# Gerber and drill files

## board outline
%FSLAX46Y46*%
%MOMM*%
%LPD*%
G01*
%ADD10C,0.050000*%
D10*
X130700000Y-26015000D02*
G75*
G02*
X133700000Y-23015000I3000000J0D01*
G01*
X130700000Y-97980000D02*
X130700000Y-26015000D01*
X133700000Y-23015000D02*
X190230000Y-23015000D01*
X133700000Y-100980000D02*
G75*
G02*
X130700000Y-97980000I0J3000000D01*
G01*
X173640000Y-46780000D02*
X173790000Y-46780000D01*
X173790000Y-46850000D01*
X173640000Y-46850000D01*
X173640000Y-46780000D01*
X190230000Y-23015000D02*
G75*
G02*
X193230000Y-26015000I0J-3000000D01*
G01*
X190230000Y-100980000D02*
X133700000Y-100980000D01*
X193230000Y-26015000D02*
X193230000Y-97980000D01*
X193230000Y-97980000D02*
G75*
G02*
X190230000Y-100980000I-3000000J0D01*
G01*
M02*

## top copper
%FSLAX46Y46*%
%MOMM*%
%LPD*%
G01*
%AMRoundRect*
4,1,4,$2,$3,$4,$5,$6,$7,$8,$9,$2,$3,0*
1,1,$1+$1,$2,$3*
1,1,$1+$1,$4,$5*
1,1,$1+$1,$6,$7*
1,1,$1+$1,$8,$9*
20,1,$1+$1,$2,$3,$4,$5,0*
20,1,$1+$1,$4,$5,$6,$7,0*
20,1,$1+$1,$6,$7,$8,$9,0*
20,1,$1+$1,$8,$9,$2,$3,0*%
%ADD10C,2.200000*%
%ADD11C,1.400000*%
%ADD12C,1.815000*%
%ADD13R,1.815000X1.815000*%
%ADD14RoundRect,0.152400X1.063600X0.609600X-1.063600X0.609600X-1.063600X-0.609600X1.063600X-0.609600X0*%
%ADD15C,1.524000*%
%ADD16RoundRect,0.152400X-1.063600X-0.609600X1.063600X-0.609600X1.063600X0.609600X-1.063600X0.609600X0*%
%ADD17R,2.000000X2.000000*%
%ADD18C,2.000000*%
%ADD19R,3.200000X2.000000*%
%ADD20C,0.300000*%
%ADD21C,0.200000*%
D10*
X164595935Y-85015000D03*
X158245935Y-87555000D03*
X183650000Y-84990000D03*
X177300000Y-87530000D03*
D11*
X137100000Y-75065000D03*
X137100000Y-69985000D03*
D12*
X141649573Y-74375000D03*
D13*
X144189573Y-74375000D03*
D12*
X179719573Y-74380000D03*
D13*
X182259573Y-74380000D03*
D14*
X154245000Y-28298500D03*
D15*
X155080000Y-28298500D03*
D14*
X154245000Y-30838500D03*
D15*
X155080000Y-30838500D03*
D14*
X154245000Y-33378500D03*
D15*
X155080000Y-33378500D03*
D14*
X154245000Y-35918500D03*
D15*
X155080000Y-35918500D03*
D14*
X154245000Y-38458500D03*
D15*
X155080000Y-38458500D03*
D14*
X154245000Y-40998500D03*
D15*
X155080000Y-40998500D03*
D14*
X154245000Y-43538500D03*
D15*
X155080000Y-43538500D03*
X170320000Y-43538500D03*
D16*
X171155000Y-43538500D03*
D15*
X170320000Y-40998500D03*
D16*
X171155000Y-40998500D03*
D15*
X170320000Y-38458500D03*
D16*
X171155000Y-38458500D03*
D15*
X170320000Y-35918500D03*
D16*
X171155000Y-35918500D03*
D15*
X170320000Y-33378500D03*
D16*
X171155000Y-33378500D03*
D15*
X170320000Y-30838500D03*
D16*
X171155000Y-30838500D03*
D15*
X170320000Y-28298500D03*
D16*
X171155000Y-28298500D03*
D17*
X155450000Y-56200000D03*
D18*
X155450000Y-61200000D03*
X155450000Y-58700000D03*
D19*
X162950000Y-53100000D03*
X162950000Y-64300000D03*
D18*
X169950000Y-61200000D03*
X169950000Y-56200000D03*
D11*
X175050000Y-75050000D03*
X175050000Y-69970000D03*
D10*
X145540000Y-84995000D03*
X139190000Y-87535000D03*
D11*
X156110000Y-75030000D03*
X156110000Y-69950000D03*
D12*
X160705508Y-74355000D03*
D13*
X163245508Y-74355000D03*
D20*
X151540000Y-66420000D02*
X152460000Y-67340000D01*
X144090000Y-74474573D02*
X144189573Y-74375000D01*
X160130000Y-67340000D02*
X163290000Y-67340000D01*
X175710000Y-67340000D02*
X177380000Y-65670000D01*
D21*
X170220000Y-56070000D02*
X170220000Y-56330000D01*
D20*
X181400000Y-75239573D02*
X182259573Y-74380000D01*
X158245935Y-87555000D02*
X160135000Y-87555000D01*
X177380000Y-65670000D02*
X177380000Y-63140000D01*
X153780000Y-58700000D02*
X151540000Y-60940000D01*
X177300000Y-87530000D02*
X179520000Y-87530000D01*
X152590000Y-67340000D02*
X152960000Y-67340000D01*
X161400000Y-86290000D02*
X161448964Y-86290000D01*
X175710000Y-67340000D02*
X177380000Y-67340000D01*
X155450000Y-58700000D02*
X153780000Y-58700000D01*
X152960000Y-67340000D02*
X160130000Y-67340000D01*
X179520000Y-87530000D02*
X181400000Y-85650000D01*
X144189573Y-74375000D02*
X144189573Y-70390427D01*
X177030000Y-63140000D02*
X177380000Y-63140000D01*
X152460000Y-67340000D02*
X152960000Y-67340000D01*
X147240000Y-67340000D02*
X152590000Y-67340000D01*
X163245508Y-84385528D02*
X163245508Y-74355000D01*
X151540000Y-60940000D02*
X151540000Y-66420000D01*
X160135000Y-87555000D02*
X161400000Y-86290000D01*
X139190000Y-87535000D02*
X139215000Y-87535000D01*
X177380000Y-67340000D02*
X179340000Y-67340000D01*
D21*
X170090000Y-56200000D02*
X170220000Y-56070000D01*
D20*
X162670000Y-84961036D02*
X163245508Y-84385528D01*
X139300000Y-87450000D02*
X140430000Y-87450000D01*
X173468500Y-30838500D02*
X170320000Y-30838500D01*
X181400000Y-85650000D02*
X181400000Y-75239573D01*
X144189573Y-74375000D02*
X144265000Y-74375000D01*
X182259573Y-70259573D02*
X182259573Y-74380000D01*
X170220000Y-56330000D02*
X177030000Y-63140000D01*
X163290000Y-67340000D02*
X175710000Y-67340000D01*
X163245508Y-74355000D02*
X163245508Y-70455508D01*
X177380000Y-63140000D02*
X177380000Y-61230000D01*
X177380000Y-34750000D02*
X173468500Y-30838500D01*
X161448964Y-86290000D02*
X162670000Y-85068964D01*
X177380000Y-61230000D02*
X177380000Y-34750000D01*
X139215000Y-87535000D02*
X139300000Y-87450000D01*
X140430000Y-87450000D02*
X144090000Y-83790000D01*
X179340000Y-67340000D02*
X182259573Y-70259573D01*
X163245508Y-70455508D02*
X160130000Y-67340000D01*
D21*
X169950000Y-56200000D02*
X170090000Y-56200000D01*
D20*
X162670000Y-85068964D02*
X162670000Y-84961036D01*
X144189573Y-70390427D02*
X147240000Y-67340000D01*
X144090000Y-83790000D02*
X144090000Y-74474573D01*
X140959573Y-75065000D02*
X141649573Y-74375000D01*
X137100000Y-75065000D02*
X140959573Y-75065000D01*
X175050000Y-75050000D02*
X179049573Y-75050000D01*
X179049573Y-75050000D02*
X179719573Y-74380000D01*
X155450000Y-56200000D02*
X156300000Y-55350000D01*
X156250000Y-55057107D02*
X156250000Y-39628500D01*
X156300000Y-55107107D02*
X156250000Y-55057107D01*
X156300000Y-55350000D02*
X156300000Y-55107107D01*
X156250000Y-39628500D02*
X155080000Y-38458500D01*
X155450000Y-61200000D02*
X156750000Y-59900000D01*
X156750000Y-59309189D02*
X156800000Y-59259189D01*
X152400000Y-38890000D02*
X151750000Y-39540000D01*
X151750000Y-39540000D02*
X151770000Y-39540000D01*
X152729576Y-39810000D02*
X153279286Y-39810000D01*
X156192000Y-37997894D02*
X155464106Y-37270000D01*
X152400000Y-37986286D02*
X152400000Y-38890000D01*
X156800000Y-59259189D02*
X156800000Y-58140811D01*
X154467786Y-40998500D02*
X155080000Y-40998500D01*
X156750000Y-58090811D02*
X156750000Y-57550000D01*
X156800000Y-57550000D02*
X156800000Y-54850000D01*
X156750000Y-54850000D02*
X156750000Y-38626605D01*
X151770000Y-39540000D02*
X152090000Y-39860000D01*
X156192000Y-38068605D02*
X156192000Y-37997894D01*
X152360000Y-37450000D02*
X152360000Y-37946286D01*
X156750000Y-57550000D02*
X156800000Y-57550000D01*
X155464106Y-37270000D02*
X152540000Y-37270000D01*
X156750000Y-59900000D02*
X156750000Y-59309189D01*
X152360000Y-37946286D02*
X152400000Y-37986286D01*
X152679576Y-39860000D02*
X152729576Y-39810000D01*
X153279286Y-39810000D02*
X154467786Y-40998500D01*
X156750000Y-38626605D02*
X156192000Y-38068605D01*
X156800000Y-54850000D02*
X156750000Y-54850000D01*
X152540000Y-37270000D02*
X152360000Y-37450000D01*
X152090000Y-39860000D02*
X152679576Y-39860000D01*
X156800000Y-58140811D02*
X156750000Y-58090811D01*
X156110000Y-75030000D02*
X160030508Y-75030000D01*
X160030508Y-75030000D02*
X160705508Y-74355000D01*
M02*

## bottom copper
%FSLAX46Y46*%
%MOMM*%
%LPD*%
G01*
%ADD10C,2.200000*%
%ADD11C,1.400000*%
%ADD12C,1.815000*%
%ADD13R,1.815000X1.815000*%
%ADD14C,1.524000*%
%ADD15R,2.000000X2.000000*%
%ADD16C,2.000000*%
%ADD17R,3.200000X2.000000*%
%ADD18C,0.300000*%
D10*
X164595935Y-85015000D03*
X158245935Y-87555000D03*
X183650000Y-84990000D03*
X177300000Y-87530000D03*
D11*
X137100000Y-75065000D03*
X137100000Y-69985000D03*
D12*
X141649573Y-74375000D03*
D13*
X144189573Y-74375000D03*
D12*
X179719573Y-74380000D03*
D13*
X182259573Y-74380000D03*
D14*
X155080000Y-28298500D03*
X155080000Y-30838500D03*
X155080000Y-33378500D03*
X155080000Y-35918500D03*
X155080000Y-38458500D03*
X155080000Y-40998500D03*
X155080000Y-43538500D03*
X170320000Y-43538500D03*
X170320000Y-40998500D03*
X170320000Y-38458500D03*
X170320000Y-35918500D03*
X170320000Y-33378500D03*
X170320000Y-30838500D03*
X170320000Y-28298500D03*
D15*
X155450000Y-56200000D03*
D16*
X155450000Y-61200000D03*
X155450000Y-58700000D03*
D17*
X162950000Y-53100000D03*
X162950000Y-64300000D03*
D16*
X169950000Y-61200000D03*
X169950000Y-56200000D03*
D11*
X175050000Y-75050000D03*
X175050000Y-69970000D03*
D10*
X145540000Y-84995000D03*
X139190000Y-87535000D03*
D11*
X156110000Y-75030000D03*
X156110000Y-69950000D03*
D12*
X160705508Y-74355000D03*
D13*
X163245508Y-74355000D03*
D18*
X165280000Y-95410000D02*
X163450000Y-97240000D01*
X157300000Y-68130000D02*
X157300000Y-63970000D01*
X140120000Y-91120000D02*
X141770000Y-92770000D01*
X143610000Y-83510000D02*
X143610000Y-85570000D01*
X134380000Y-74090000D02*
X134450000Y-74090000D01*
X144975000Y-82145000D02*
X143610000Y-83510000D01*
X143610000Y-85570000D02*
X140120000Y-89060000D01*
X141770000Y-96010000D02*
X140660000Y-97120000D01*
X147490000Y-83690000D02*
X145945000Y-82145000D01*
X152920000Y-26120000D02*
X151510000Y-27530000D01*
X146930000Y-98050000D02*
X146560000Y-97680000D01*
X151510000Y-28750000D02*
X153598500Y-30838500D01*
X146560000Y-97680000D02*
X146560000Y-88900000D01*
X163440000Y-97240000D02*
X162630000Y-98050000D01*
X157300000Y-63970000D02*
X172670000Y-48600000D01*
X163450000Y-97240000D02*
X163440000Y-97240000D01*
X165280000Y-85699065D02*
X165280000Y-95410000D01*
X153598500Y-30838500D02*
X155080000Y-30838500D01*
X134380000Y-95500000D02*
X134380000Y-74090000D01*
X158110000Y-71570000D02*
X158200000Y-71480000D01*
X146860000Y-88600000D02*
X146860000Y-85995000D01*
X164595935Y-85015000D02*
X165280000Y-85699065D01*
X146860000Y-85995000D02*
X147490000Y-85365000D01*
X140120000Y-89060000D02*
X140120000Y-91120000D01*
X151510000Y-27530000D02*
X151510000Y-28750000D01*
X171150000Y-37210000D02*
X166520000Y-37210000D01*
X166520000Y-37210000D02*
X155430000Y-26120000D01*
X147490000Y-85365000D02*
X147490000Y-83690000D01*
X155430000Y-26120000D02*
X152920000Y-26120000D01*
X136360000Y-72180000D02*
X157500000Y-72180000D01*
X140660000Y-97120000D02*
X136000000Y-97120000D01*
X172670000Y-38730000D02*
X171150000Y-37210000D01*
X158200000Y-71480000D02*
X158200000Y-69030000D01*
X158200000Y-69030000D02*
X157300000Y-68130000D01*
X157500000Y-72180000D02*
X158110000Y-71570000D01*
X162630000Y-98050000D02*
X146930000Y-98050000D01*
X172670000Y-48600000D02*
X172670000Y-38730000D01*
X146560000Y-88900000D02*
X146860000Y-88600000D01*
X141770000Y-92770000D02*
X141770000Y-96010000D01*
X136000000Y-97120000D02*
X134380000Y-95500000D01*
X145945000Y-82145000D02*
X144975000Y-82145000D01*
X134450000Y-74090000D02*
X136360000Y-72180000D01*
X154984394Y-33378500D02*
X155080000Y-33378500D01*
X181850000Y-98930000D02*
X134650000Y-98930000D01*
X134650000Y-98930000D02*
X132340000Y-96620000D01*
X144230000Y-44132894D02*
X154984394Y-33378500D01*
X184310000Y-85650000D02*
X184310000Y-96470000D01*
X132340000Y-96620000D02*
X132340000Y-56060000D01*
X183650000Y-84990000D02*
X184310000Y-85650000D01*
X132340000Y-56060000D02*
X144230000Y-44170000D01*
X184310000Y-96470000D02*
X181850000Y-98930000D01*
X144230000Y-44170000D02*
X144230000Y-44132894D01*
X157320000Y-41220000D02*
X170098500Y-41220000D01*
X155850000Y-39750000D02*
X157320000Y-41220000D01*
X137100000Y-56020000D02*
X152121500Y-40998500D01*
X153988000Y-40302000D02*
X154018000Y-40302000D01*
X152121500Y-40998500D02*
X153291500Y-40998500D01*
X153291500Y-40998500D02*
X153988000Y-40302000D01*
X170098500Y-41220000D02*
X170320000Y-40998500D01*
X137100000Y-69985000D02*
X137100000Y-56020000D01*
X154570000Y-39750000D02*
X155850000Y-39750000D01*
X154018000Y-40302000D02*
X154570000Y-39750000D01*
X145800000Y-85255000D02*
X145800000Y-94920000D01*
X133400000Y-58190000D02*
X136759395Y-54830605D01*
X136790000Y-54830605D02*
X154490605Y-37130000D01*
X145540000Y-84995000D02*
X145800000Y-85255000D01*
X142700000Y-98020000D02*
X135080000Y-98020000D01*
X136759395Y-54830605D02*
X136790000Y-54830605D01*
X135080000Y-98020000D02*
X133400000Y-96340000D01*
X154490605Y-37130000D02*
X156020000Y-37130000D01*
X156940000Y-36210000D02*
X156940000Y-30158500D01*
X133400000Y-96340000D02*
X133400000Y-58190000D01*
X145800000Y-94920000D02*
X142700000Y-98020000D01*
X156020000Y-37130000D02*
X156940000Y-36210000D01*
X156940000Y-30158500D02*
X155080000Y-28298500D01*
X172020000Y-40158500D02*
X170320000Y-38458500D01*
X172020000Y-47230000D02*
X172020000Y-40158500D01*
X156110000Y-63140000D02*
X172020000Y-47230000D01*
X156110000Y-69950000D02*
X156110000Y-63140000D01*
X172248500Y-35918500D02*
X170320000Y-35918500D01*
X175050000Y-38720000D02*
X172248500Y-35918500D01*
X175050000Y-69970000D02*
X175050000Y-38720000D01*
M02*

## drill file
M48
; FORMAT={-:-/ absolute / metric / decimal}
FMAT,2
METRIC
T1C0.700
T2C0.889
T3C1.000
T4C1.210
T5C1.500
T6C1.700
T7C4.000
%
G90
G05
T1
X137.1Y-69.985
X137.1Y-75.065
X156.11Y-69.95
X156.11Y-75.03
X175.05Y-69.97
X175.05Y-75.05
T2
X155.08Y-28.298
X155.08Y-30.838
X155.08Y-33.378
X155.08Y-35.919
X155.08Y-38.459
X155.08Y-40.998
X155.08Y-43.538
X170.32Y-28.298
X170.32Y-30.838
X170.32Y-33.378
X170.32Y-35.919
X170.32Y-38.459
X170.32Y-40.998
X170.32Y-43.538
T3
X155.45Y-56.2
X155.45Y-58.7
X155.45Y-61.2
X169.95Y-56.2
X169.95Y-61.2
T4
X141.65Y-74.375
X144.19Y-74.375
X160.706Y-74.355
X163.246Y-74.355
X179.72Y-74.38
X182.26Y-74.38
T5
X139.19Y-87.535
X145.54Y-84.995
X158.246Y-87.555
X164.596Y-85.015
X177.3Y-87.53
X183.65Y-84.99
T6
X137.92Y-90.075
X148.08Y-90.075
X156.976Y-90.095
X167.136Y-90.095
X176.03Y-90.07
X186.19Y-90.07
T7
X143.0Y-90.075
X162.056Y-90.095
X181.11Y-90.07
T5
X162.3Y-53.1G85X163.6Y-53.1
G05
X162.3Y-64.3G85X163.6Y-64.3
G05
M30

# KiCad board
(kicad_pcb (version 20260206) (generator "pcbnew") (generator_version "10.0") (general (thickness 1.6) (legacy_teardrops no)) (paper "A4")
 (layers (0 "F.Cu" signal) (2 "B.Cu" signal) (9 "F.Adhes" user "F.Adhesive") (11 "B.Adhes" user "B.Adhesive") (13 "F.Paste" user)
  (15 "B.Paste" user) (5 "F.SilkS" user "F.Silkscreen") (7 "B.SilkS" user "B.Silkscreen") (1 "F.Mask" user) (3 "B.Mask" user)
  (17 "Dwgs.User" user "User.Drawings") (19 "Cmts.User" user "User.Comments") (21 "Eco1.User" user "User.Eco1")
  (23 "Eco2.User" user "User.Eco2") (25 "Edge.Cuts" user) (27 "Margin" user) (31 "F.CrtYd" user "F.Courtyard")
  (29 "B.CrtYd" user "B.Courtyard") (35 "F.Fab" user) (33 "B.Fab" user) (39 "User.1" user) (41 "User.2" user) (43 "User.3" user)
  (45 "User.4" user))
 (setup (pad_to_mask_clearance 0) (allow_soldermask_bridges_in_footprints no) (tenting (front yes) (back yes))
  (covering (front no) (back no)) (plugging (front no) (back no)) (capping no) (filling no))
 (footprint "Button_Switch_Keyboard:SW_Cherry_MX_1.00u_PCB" (layer "F.Cu") (at 164.595935 85.015)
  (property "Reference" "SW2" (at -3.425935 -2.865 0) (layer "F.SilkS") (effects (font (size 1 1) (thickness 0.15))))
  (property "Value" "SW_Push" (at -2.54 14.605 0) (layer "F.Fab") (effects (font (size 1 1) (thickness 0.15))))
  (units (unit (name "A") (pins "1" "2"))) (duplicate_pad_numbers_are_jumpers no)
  (pad "" np_thru_hole circle (at -7.62 5.08) (size 1.7 1.7) (drill 1.7) (layers "*.Cu" "*.Mask"))
  (pad "" np_thru_hole circle (at -2.54 5.08) (size 4 4) (drill 4) (layers "*.Cu" "*.Mask"))
  (pad "" np_thru_hole circle (at 2.54 5.08) (size 1.7 1.7) (drill 1.7) (layers "*.Cu" "*.Mask"))
  (pad "1" thru_hole circle (at 0 0) (size 2.2 2.2) (drill 1.5) (layers "*.Cu" "*.Mask") (remove_unused_layers no) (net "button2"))
  (pad "2" thru_hole circle (at -6.35 2.54) (size 2.2 2.2) (drill 1.5) (layers "*.Cu" "*.Mask") (remove_unused_layers no) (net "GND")))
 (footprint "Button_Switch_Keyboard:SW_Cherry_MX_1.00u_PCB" (layer "F.Cu") (at 183.65 84.99)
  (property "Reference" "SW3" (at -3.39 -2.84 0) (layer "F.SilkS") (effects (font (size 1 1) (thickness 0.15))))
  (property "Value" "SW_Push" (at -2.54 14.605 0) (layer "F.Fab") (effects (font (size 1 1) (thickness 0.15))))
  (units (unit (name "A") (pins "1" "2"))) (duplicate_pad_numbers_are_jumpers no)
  (pad "" np_thru_hole circle (at -7.62 5.08) (size 1.7 1.7) (drill 1.7) (layers "*.Cu" "*.Mask"))
  (pad "" np_thru_hole circle (at -2.54 5.08) (size 4 4) (drill 4) (layers "*.Cu" "*.Mask"))
  (pad "" np_thru_hole circle (at 2.54 5.08) (size 1.7 1.7) (drill 1.7) (layers "*.Cu" "*.Mask"))
  (pad "1" thru_hole circle (at 0 0) (size 2.2 2.2) (drill 1.5) (layers "*.Cu" "*.Mask") (remove_unused_layers no) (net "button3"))
  (pad "2" thru_hole circle (at -6.35 2.54) (size 2.2 2.2) (drill 1.5) (layers "*.Cu" "*.Mask") (remove_unused_layers no) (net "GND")))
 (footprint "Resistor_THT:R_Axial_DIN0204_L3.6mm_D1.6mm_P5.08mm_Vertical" (layer "F.Cu") (at 137.1 75.065 90)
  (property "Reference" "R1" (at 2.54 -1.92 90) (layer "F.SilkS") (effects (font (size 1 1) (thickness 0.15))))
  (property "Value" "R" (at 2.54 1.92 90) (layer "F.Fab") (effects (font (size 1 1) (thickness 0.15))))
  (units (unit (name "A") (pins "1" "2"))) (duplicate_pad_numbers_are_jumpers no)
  (pad "1" thru_hole circle (at 0 0 90) (size 1.4 1.4) (drill 0.7) (layers "*.Cu" "*.Mask") (remove_unused_layers no) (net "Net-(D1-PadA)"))
  (pad "2" thru_hole circle (at 5.08 0 90) (size 1.4 1.4) (drill 0.7) (layers "*.Cu" "*.Mask") (remove_unused_layers no) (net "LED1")))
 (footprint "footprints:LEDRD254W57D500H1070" (layer "F.Cu") (at 142.919573 74.375 180)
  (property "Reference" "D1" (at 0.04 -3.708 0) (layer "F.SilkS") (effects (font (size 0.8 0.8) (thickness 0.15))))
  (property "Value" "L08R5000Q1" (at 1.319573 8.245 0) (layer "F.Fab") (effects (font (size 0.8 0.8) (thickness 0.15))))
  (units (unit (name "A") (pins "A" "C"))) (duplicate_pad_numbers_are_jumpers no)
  (pad "A" thru_hole circle (at 1.27 0 180) (size 1.815 1.815) (drill 1.21) (layers "*.Cu" "*.Mask") (remove_unused_layers no)
   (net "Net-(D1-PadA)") (solder_mask_margin 0.102))
  (pad "C" thru_hole rect (at -1.27 0 180) (size 1.815 1.815) (drill 1.21) (layers "*.Cu" "*.Mask") (remove_unused_layers no) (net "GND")
   (solder_mask_margin 0.102)))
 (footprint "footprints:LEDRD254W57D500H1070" (layer "F.Cu") (at 180.989573 74.38 180)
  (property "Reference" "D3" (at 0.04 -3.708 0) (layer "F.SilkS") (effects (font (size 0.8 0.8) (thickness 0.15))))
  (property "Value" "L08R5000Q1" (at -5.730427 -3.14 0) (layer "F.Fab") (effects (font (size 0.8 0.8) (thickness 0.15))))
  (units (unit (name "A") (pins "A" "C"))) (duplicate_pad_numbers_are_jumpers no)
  (pad "A" thru_hole circle (at 1.27 0 180) (size 1.815 1.815) (drill 1.21) (layers "*.Cu" "*.Mask") (remove_unused_layers no)
   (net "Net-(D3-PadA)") (solder_mask_margin 0.102))
  (pad "C" thru_hole rect (at -1.27 0 180) (size 1.815 1.815) (drill 1.21) (layers "*.Cu" "*.Mask") (remove_unused_layers no) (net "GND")
   (solder_mask_margin 0.102)))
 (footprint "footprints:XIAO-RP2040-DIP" (layer "F.Cu") (at 162.7 35.9185 90)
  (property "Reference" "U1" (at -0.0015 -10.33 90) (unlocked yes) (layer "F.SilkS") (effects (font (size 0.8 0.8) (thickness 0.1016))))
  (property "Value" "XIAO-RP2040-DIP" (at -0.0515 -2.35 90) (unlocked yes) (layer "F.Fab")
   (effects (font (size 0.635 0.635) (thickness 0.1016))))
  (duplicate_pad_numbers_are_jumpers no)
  (pad "1" smd roundrect (at 7.62 -8.455 180) (size 2.432 1.524) (layers "F.Cu" "F.Mask") (roundrect_rratio 0.1) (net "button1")
   (thermal_bridge_angle 45))
  (pad "1" thru_hole circle (at 7.62 -7.62 180) (size 1.524 1.524) (drill 0.889) (layers "*.Cu" "*.Mask") (remove_unused_layers no)
   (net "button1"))
  (pad "2" smd roundrect (at 5.08 -8.455 180) (size 2.432 1.524) (layers "F.Cu" "F.Mask") (roundrect_rratio 0.1) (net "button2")
   (thermal_bridge_angle 45))
  (pad "2" thru_hole circle (at 5.08 -7.62 180) (size 1.524 1.524) (drill 0.889) (layers "*.Cu" "*.Mask") (remove_unused_layers no)
   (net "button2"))
  (pad "3" smd roundrect (at 2.54 -8.455 180) (size 2.432 1.524) (layers "F.Cu" "F.Mask") (roundrect_rratio 0.1) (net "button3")
   (thermal_bridge_angle 45))
  (pad "3" thru_hole circle (at 2.54 -7.62 180) (size 1.524 1.524) (drill 0.889) (layers "*.Cu" "*.Mask") (remove_unused_layers no)
   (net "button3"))
  (pad "4" smd roundrect (at 0 -8.455 180) (size 2.432 1.524) (layers "F.Cu" "F.Mask") (roundrect_rratio 0.1)
   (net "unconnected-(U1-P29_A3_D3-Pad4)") (thermal_bridge_angle 45))
  (pad "4" thru_hole circle (at 0 -7.62 180) (size 1.524 1.524) (drill 0.889) (layers "*.Cu" "*.Mask") (remove_unused_layers no)
   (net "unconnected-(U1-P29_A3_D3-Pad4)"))
  (pad "5" smd roundrect (at -2.54 -8.455 180) (size 2.432 1.524) (layers "F.Cu" "F.Mask") (roundrect_rratio 0.1) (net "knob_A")
   (thermal_bridge_angle 45))
  (pad "5" thru_hole circle (at -2.54 -7.62 180) (size 1.524 1.524) (drill 0.889) (layers "*.Cu" "*.Mask") (remove_unused_layers no)
   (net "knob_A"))
  (pad "6" smd roundrect (at -5.08 -8.455 180) (size 2.432 1.524) (layers "F.Cu" "F.Mask") (roundrect_rratio 0.1) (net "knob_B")
   (thermal_bridge_angle 45))
  (pad "6" thru_hole circle (at -5.08 -7.62 180) (size 1.524 1.524) (drill 0.889) (layers "*.Cu" "*.Mask") (remove_unused_layers no)
   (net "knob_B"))
  (pad "7" smd roundrect (at -7.62 -8.455 180) (size 2.432 1.524) (layers "F.Cu" "F.Mask") (roundrect_rratio 0.1)
   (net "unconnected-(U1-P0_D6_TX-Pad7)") (thermal_bridge_angle 45))
  (pad "7" thru_hole circle (at -7.62 -7.62 180) (size 1.524 1.524) (drill 0.889) (layers "*.Cu" "*.Mask") (remove_unused_layers no)
   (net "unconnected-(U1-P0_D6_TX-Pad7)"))
  (pad "8" thru_hole circle (at -7.62 7.62) (size 1.524 1.524) (drill 0.889) (layers "*.Cu" "*.Mask") (remove_unused_layers no)
   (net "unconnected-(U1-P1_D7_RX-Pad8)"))
  (pad "8" smd roundrect (at -7.62 8.455) (size 2.432 1.524) (layers "F.Cu" "F.Mask") (roundrect_rratio 0.1)
   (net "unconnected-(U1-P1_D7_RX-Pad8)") (thermal_bridge_angle 45))
  (pad "9" thru_hole circle (at -5.08 7.62) (size 1.524 1.524) (drill 0.889) (layers "*.Cu" "*.Mask") (remove_unused_layers no) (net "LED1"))
  (pad "9" smd roundrect (at -5.08 8.455) (size 2.432 1.524) (layers "F.Cu" "F.Mask") (roundrect_rratio 0.1) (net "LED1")
   (thermal_bridge_angle 45))
  (pad "10" thru_hole circle (at -2.54 7.62) (size 1.524 1.524) (drill 0.889) (layers "*.Cu" "*.Mask") (remove_unused_layers no)
   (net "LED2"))
  (pad "10" smd roundrect (at -2.54 8.455) (size 2.432 1.524) (layers "F.Cu" "F.Mask") (roundrect_rratio 0.1) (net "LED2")
   (thermal_bridge_angle 45))
  (pad "11" thru_hole circle (at 0 7.62) (size 1.524 1.524) (drill 0.889) (layers "*.Cu" "*.Mask") (remove_unused_layers no) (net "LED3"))
  (pad "11" smd roundrect (at 0 8.455) (size 2.432 1.524) (layers "F.Cu" "F.Mask") (roundrect_rratio 0.1) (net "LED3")
   (thermal_bridge_angle 45))
  (pad "12" thru_hole circle (at 2.54 7.62) (size 1.524 1.524) (drill 0.889) (layers "*.Cu" "*.Mask") (remove_unused_layers no)
   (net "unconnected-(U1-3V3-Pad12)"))
  (pad "12" smd roundrect (at 2.54 8.455) (size 2.432 1.524) (layers "F.Cu" "F.Mask") (roundrect_rratio 0.1)
   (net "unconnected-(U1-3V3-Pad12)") (thermal_bridge_angle 45))
  (pad "13" thru_hole circle (at 5.08 7.62) (size 1.524 1.524) (drill 0.889) (layers "*.Cu" "*.Mask") (remove_unused_layers no) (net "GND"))
  (pad "13" smd roundrect (at 5.08 8.455) (size 2.432 1.524) (layers "F.Cu" "F.Mask") (roundrect_rratio 0.1) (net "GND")
   (thermal_bridge_angle 45))
  (pad "14" thru_hole circle (at 7.62 7.62) (size 1.524 1.524) (drill 0.889) (layers "*.Cu" "*.Mask") (remove_unused_layers no)
   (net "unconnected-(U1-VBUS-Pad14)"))
  (pad "14" smd roundrect (at 7.62 8.455) (size 2.432 1.524) (layers "F.Cu" "F.Mask") (roundrect_rratio 0.1)
   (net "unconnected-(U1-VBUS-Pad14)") (thermal_bridge_angle 45)))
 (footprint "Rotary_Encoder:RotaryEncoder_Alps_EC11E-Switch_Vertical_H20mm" (layer "F.Cu") (at 155.45 56.2)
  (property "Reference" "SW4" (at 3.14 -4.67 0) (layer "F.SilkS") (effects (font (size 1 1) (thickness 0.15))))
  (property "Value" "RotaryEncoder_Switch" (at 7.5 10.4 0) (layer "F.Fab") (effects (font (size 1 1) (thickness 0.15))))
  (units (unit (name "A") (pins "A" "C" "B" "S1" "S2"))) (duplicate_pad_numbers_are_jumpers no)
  (pad "A" thru_hole rect (at 0 0) (size 2 2) (drill 1) (layers "*.Cu" "*.Mask") (remove_unused_layers no) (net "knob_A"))
  (pad "B" thru_hole circle (at 0 5) (size 2 2) (drill 1) (layers "*.Cu" "*.Mask") (remove_unused_layers no) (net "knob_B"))
  (pad "C" thru_hole circle (at 0 2.5) (size 2 2) (drill 1) (layers "*.Cu" "*.Mask") (remove_unused_layers no) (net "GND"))
  (pad "MP" thru_hole rect (at 7.5 -3.1) (size 3.2 2) (drill oval 2.8 1.5) (layers "*.Cu" "*.Mask") (remove_unused_layers no))
  (pad "MP" thru_hole rect (at 7.5 8.1) (size 3.2 2) (drill oval 2.8 1.5) (layers "*.Cu" "*.Mask") (remove_unused_layers no))
  (pad "S1" thru_hole circle (at 14.5 5) (size 2 2) (drill 1) (layers "*.Cu" "*.Mask") (remove_unused_layers no) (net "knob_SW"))
  (pad "S2" thru_hole circle (at 14.5 0) (size 2 2) (drill 1) (layers "*.Cu" "*.Mask") (remove_unused_layers no) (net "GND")))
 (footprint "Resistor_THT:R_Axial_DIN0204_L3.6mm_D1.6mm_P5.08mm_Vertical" (layer "F.Cu") (at 175.05 75.05 90)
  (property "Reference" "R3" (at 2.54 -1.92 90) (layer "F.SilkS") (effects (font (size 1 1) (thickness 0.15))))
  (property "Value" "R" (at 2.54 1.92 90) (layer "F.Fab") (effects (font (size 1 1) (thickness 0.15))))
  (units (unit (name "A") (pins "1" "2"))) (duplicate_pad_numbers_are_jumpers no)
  (pad "1" thru_hole circle (at 0 0 90) (size 1.4 1.4) (drill 0.7) (layers "*.Cu" "*.Mask") (remove_unused_layers no) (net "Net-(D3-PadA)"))
  (pad "2" thru_hole circle (at 5.08 0 90) (size 1.4 1.4) (drill 0.7) (layers "*.Cu" "*.Mask") (remove_unused_layers no) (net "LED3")))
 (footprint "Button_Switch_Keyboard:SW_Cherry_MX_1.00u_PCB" (layer "F.Cu") (at 145.54 84.995)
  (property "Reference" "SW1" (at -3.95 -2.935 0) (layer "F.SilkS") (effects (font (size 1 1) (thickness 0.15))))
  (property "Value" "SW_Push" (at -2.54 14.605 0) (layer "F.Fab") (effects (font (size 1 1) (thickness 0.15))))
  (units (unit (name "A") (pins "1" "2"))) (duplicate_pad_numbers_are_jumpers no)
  (pad "" np_thru_hole circle (at -7.62 5.08) (size 1.7 1.7) (drill 1.7) (layers "*.Cu" "*.Mask"))
  (pad "" np_thru_hole circle (at -2.54 5.08) (size 4 4) (drill 4) (layers "*.Cu" "*.Mask"))
  (pad "" np_thru_hole circle (at 2.54 5.08) (size 1.7 1.7) (drill 1.7) (layers "*.Cu" "*.Mask"))
  (pad "1" thru_hole circle (at 0 0) (size 2.2 2.2) (drill 1.5) (layers "*.Cu" "*.Mask") (remove_unused_layers no) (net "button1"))
  (pad "2" thru_hole circle (at -6.35 2.54) (size 2.2 2.2) (drill 1.5) (layers "*.Cu" "*.Mask") (remove_unused_layers no) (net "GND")))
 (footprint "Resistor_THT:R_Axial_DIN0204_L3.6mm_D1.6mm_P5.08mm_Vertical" (layer "F.Cu") (at 156.11 75.03 90)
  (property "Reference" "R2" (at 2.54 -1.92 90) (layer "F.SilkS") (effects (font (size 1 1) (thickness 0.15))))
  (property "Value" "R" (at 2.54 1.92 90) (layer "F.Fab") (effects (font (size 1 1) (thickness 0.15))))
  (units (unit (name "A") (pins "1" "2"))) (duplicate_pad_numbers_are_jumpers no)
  (pad "1" thru_hole circle (at 0 0 90) (size 1.4 1.4) (drill 0.7) (layers "*.Cu" "*.Mask") (remove_unused_layers no) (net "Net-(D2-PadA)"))
  (pad "2" thru_hole circle (at 5.08 0 90) (size 1.4 1.4) (drill 0.7) (layers "*.Cu" "*.Mask") (remove_unused_layers no) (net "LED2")))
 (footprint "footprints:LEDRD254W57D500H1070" (layer "F.Cu") (at 161.975508 74.355 180)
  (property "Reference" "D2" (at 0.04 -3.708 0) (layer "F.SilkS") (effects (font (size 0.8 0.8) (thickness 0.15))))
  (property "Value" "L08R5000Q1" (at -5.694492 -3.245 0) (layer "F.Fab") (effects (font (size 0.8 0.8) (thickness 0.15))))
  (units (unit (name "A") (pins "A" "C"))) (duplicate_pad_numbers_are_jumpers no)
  (pad "A" thru_hole circle (at 1.27 0 180) (size 1.815 1.815) (drill 1.21) (layers "*.Cu" "*.Mask") (remove_unused_layers no)
   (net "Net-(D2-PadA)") (solder_mask_margin 0.102))
  (pad "C" thru_hole rect (at -1.27 0 180) (size 1.815 1.815) (drill 1.21) (layers "*.Cu" "*.Mask") (remove_unused_layers no) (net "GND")
   (solder_mask_margin 0.102)))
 (gr_arc (start 130.7 26.015) (mid 131.57868 23.89368) (end 133.7 23.015) (stroke (width 0.05) (type default)) (layer "Edge.Cuts"))
 (gr_line (start 130.7 97.98) (end 130.7 26.015) (stroke (width 0.05) (type default)) (layer "Edge.Cuts"))
 (gr_line (start 133.7 23.015) (end 190.23 23.015) (stroke (width 0.05) (type default)) (layer "Edge.Cuts"))
 (gr_arc (start 133.7 100.98) (mid 131.57868 100.10132) (end 130.7 97.98) (stroke (width 0.05) (type default)) (layer "Edge.Cuts"))
 (gr_rect (start 173.64 46.78) (end 173.79 46.85) (stroke (width 0.05) (type default)) (fill no) (layer "Edge.Cuts"))
 (gr_arc (start 190.23 23.015) (mid 192.35132 23.89368) (end 193.23 26.015) (stroke (width 0.05) (type default)) (layer "Edge.Cuts"))
 (gr_line (start 190.23 100.98) (end 133.7 100.98) (stroke (width 0.05) (type default)) (layer "Edge.Cuts"))
 (gr_line (start 193.23 26.015) (end 193.23 97.98) (stroke (width 0.05) (type default)) (layer "Edge.Cuts"))
 (gr_arc (start 193.23 97.98) (mid 192.35132 100.10132) (end 190.23 100.98) (stroke (width 0.05) (type default)) (layer "Edge.Cuts"))
 (segment (start 165.28 95.41) (end 163.45 97.24) (width 0.3) (layer "B.Cu") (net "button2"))
 (segment (start 157.3 68.13) (end 157.3 63.97) (width 0.3) (layer "B.Cu") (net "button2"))
 (segment (start 140.12 91.12) (end 141.77 92.77) (width 0.3) (layer "B.Cu") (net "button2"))
 (segment (start 143.61 83.51) (end 143.61 85.57) (width 0.3) (layer "B.Cu") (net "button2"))
 (segment (start 134.38 74.09) (end 134.45 74.09) (width 0.3) (layer "B.Cu") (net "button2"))
 (segment (start 144.975 82.145) (end 143.61 83.51) (width 0.3) (layer "B.Cu") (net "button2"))
 (segment (start 143.61 85.57) (end 140.12 89.06) (width 0.3) (layer "B.Cu") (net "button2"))
 (segment (start 141.77 96.01) (end 140.66 97.12) (width 0.3) (layer "B.Cu") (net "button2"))
 (segment (start 147.49 83.69) (end 145.945 82.145) (width 0.3) (layer "B.Cu") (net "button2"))
 (segment (start 152.92 26.12) (end 151.51 27.53) (width 0.3) (layer "B.Cu") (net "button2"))
 (segment (start 146.93 98.05) (end 146.56 97.68) (width 0.3) (layer "B.Cu") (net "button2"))
 (segment (start 151.51 28.75) (end 153.5985 30.8385) (width 0.3) (layer "B.Cu") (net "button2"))
 (segment (start 146.56 97.68) (end 146.56 88.9) (width 0.3) (layer "B.Cu") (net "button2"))
 (segment (start 163.44 97.24) (end 162.63 98.05) (width 0.3) (layer "B.Cu") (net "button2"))
 (segment (start 157.3 63.97) (end 172.67 48.6) (width 0.3) (layer "B.Cu") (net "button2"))
 (segment (start 163.45 97.24) (end 163.44 97.24) (width 0.3) (layer "B.Cu") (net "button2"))
 (segment (start 165.28 85.699065) (end 165.28 95.41) (width 0.3) (layer "B.Cu") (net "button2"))
 (segment (start 153.5985 30.8385) (end 155.08 30.8385) (width 0.3) (layer "B.Cu") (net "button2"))
 (segment (start 134.38 95.5) (end 134.38 74.09) (width 0.3) (layer "B.Cu") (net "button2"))
 (segment (start 158.11 71.57) (end 158.2 71.48) (width 0.3) (layer "B.Cu") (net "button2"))
 (segment (start 146.86 88.6) (end 146.86 85.995) (width 0.3) (layer "B.Cu") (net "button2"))
 (segment (start 164.595935 85.015) (end 165.28 85.699065) (width 0.3) (layer "B.Cu") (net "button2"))
 (segment (start 146.86 85.995) (end 147.49 85.365) (width 0.3) (layer "B.Cu") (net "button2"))
 (segment (start 140.12 89.06) (end 140.12 91.12) (width 0.3) (layer "B.Cu") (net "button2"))
 (segment (start 151.51 27.53) (end 151.51 28.75) (width 0.3) (layer "B.Cu") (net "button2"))
 (segment (start 171.15 37.21) (end 166.52 37.21) (width 0.3) (layer "B.Cu") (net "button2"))
 (segment (start 166.52 37.21) (end 155.43 26.12) (width 0.3) (layer "B.Cu") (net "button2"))
 (segment (start 147.49 85.365) (end 147.49 83.69) (width 0.3) (layer "B.Cu") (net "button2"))
 (segment (start 155.43 26.12) (end 152.92 26.12) (width 0.3) (layer "B.Cu") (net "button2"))
 (segment (start 136.36 72.18) (end 157.5 72.18) (width 0.3) (layer "B.Cu") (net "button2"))
 (segment (start 140.66 97.12) (end 136 97.12) (width 0.3) (layer "B.Cu") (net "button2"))
 (segment (start 172.67 38.73) (end 171.15 37.21) (width 0.3) (layer "B.Cu") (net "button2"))
 (segment (start 158.2 71.48) (end 158.2 69.03) (width 0.3) (layer "B.Cu") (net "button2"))
 (segment (start 158.2 69.03) (end 157.3 68.13) (width 0.3) (layer "B.Cu") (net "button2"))
 (segment (start 157.5 72.18) (end 158.11 71.57) (width 0.3) (layer "B.Cu") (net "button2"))
 (segment (start 162.63 98.05) (end 146.93 98.05) (width 0.3) (layer "B.Cu") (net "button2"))
 (segment (start 172.67 48.6) (end 172.67 38.73) (width 0.3) (layer "B.Cu") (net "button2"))
 (segment (start 146.56 88.9) (end 146.86 88.6) (width 0.3) (layer "B.Cu") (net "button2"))
 (segment (start 141.77 92.77) (end 141.77 96.01) (width 0.3) (layer "B.Cu") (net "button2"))
 (segment (start 136 97.12) (end 134.38 95.5) (width 0.3) (layer "B.Cu") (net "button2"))
 (segment (start 145.945 82.145) (end 144.975 82.145) (width 0.3) (layer "B.Cu") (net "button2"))
 (segment (start 134.45 74.09) (end 136.36 72.18) (width 0.3) (layer "B.Cu") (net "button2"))
 (segment (start 151.54 66.42) (end 152.46 67.34) (width 0.3) (layer "F.Cu") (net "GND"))
 (segment (start 144.09 74.474573) (end 144.189573 74.375) (width 0.3) (layer "F.Cu") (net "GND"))
 (segment (start 160.13 67.34) (end 163.29 67.34) (width 0.3) (layer "F.Cu") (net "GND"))
 (segment (start 175.71 67.34) (end 177.38 65.67) (width 0.3) (layer "F.Cu") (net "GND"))
 (segment (start 170.22 56.07) (end 170.22 56.33) (width 0.2) (layer "F.Cu") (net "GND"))
 (segment (start 181.4 75.239573) (end 182.259573 74.38) (width 0.3) (layer "F.Cu") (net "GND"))
 (segment (start 158.245935 87.555) (end 160.135 87.555) (width 0.3) (layer "F.Cu") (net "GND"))
 (segment (start 177.38 65.67) (end 177.38 63.14) (width 0.3) (layer "F.Cu") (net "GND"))
 (segment (start 153.78 58.7) (end 151.54 60.94) (width 0.3) (layer "F.Cu") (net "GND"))
 (segment (start 177.3 87.53) (end 179.52 87.53) (width 0.3) (layer "F.Cu") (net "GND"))
 (segment (start 152.59 67.34) (end 152.96 67.34) (width 0.3) (layer "F.Cu") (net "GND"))
 (segment (start 161.4 86.29) (end 161.448964 86.29) (width 0.3) (layer "F.Cu") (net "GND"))
 (segment (start 175.71 67.34) (end 177.38 67.34) (width 0.3) (layer "F.Cu") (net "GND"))
 (segment (start 155.45 58.7) (end 153.78 58.7) (width 0.3) (layer "F.Cu") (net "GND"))
 (segment (start 152.96 67.34) (end 160.13 67.34) (width 0.3) (layer "F.Cu") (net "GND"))
 (segment (start 179.52 87.53) (end 181.4 85.65) (width 0.3) (layer "F.Cu") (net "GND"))
 (segment (start 144.189573 74.375) (end 144.189573 70.390427) (width 0.3) (layer "F.Cu") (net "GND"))
 (segment (start 177.03 63.14) (end 177.38 63.14) (width 0.3) (layer "F.Cu") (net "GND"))
 (segment (start 152.46 67.34) (end 152.96 67.34) (width 0.3) (layer "F.Cu") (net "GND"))
 (segment (start 147.24 67.34) (end 152.59 67.34) (width 0.3) (layer "F.Cu") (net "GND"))
 (segment (start 163.245508 84.385528) (end 163.245508 74.355) (width 0.3) (layer "F.Cu") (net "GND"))
 (segment (start 151.54 60.94) (end 151.54 66.42) (width 0.3) (layer "F.Cu") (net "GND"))
 (segment (start 160.135 87.555) (end 161.4 86.29) (width 0.3) (layer "F.Cu") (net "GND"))
 (segment (start 139.19 87.535) (end 139.215 87.535) (width 0.3) (layer "F.Cu") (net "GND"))
 (segment (start 177.38 67.34) (end 179.34 67.34) (width 0.3) (layer "F.Cu") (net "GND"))
 (segment (start 170.09 56.2) (end 170.22 56.07) (width 0.2) (layer "F.Cu") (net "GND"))
 (segment (start 162.67 84.961036) (end 163.245508 84.385528) (width 0.3) (layer "F.Cu") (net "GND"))
 (segment (start 139.3 87.45) (end 140.43 87.45) (width 0.3) (layer "F.Cu") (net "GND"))
 (segment (start 173.4685 30.8385) (end 170.32 30.8385) (width 0.3) (layer "F.Cu") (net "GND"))
 (segment (start 181.4 85.65) (end 181.4 75.239573) (width 0.3) (layer "F.Cu") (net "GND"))
 (segment (start 144.189573 74.375) (end 144.265 74.375) (width 0.3) (layer "F.Cu") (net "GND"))
 (segment (start 182.259573 70.259573) (end 182.259573 74.38) (width 0.3) (layer "F.Cu") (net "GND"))
 (segment (start 170.22 56.33) (end 177.03 63.14) (width 0.3) (layer "F.Cu") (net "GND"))
 (segment (start 163.29 67.34) (end 175.71 67.34) (width 0.3) (layer "F.Cu") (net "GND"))
 (segment (start 163.245508 74.355) (end 163.245508 70.455508) (width 0.3) (layer "F.Cu") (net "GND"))
 (segment (start 177.38 63.14) (end 177.38 61.23) (width 0.3) (layer "F.Cu") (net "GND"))
 (segment (start 177.38 34.75) (end 173.4685 30.8385) (width 0.3) (layer "F.Cu") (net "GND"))
 (segment (start 161.448964 86.29) (end 162.67 85.068964) (width 0.3) (layer "F.Cu") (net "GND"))
 (segment (start 177.38 61.23) (end 177.38 34.75) (width 0.3) (layer "F.Cu") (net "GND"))
 (segment (start 139.215 87.535) (end 139.3 87.45) (width 0.3) (layer "F.Cu") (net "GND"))
 (segment (start 140.43 87.45) (end 144.09 83.79) (width 0.3) (layer "F.Cu") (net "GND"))
 (segment (start 179.34 67.34) (end 182.259573 70.259573) (width 0.3) (layer "F.Cu") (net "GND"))
 (segment (start 163.245508 70.455508) (end 160.13 67.34) (width 0.3) (layer "F.Cu") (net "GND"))
 (segment (start 169.95 56.2) (end 170.09 56.2) (width 0.2) (layer "F.Cu") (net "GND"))
 (segment (start 162.67 85.068964) (end 162.67 84.961036) (width 0.3) (layer "F.Cu") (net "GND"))
 (segment (start 144.189573 70.390427) (end 147.24 67.34) (width 0.3) (layer "F.Cu") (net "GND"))
 (segment (start 144.09 83.79) (end 144.09 74.474573) (width 0.3) (layer "F.Cu") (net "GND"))
 (segment (start 154.984394 33.3785) (end 155.08 33.3785) (width 0.3) (layer "B.Cu") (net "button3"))
 (segment (start 181.85 98.93) (end 134.65 98.93) (width 0.3) (layer "B.Cu") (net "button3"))
 (segment (start 134.65 98.93) (end 132.34 96.62) (width 0.3) (layer "B.Cu") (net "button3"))
 (segment (start 144.23 44.132894) (end 154.984394 33.3785) (width 0.3) (layer "B.Cu") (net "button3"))
 (segment (start 184.31 85.65) (end 184.31 96.47) (width 0.3) (layer "B.Cu") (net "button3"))
 (segment (start 132.34 96.62) (end 132.34 56.06) (width 0.3) (layer "B.Cu") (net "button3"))
 (segment (start 183.65 84.99) (end 184.31 85.65) (width 0.3) (layer "B.Cu") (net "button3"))
 (segment (start 132.34 56.06) (end 144.23 44.17) (width 0.3) (layer "B.Cu") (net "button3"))
 (segment (start 184.31 96.47) (end 181.85 98.93) (width 0.3) (layer "B.Cu") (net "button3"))
 (segment (start 144.23 44.17) (end 144.23 44.132894) (width 0.3) (layer "B.Cu") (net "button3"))
 (segment (start 140.959573 75.065) (end 141.649573 74.375) (width 0.3) (layer "F.Cu") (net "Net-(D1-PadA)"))
 (segment (start 137.1 75.065) (end 140.959573 75.065) (width 0.3) (layer "F.Cu") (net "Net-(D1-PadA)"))
 (segment (start 157.32 41.22) (end 170.0985 41.22) (width 0.3) (layer "B.Cu") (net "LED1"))
 (segment (start 155.85 39.75) (end 157.32 41.22) (width 0.3) (layer "B.Cu") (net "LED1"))
 (segment (start 137.1 56.02) (end 152.1215 40.9985) (width 0.3) (layer "B.Cu") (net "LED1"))
 (segment (start 153.988 40.302) (end 154.018 40.302) (width 0.3) (layer "B.Cu") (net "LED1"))
 (segment (start 152.1215 40.9985) (end 153.2915 40.9985) (width 0.3) (layer "B.Cu") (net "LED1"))
 (segment (start 153.2915 40.9985) (end 153.988 40.302) (width 0.3) (layer "B.Cu") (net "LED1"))
 (segment (start 170.0985 41.22) (end 170.32 40.9985) (width 0.3) (layer "B.Cu") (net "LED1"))
 (segment (start 137.1 69.985) (end 137.1 56.02) (width 0.3) (layer "B.Cu") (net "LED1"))
 (segment (start 154.57 39.75) (end 155.85 39.75) (width 0.3) (layer "B.Cu") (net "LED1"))
 (segment (start 154.018 40.302) (end 154.57 39.75) (width 0.3) (layer "B.Cu") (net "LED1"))
 (segment (start 175.05 75.05) (end 179.049573 75.05) (width 0.3) (layer "F.Cu") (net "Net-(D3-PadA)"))
 (segment (start 179.049573 75.05) (end 179.719573 74.38) (width 0.3) (layer "F.Cu") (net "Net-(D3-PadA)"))
 (segment (start 145.8 85.255) (end 145.8 94.92) (width 0.3) (layer "B.Cu") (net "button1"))
 (segment (start 133.4 58.19) (end 136.759395 54.830605) (width 0.3) (layer "B.Cu") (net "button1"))
 (segment (start 136.79 54.830605) (end 154.490605 37.13) (width 0.3) (layer "B.Cu") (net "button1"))
 (segment (start 145.54 84.995) (end 145.8 85.255) (width 0.3) (layer "B.Cu") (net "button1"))
 (segment (start 142.7 98.02) (end 135.08 98.02) (width 0.3) (layer "B.Cu") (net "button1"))
 (segment (start 136.759395 54.830605) (end 136.79 54.830605) (width 0.3) (layer "B.Cu") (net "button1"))
 (segment (start 135.08 98.02) (end 133.4 96.34) (width 0.3) (layer "B.Cu") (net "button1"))
 (segment (start 154.490605 37.13) (end 156.02 37.13) (width 0.3) (layer "B.Cu") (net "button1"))
 (segment (start 156.94 36.21) (end 156.94 30.1585) (width 0.3) (layer "B.Cu") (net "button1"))
 (segment (start 133.4 96.34) (end 133.4 58.19) (width 0.3) (layer "B.Cu") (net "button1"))
 (segment (start 145.8 94.92) (end 142.7 98.02) (width 0.3) (layer "B.Cu") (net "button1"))
 (segment (start 156.02 37.13) (end 156.94 36.21) (width 0.3) (layer "B.Cu") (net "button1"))
 (segment (start 156.94 30.1585) (end 155.08 28.2985) (width 0.3) (layer "B.Cu") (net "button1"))
 (segment (start 155.45 56.2) (end 156.3 55.35) (width 0.3) (layer "F.Cu") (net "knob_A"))
 (segment (start 156.25 55.057107) (end 156.25 39.6285) (width 0.3) (layer "F.Cu") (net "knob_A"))
 (segment (start 156.3 55.107107) (end 156.25 55.057107) (width 0.3) (layer "F.Cu") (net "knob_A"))
 (segment (start 156.3 55.35) (end 156.3 55.107107) (width 0.3) (layer "F.Cu") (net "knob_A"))
 (segment (start 156.25 39.6285) (end 155.08 38.4585) (width 0.3) (layer "F.Cu") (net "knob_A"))
 (segment (start 155.45 61.2) (end 156.75 59.9) (width 0.3) (layer "F.Cu") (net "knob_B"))
 (segment (start 156.75 59.309189) (end 156.8 59.259189) (width 0.3) (layer "F.Cu") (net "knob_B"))
 (segment (start 152.4 38.89) (end 151.75 39.54) (width 0.3) (layer "F.Cu") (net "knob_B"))
 (segment (start 151.75 39.54) (end 151.77 39.54) (width 0.3) (layer "F.Cu") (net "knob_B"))
 (segment (start 152.729576 39.81) (end 153.279286 39.81) (width 0.3) (layer "F.Cu") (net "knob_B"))
 (segment (start 156.192 37.997894) (end 155.464106 37.27) (width 0.3) (layer "F.Cu") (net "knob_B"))
 (segment (start 152.4 37.986286) (end 152.4 38.89) (width 0.3) (layer "F.Cu") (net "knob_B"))
 (segment (start 156.8 59.259189) (end 156.8 58.140811) (width 0.3) (layer "F.Cu") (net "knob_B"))
 (segment (start 154.467786 40.9985) (end 155.08 40.9985) (width 0.3) (layer "F.Cu") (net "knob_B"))
 (segment (start 156.75 58.090811) (end 156.75 57.55) (width 0.3) (layer "F.Cu") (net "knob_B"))
 (segment (start 156.8 57.55) (end 156.8 54.85) (width 0.3) (layer "F.Cu") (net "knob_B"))
 (segment (start 156.75 54.85) (end 156.75 38.626605) (width 0.3) (layer "F.Cu") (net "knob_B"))
 (segment (start 151.77 39.54) (end 152.09 39.86) (width 0.3) (layer "F.Cu") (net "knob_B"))
 (segment (start 156.192 38.068605) (end 156.192 37.997894) (width 0.3) (layer "F.Cu") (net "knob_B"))
 (segment (start 152.36 37.45) (end 152.36 37.946286) (width 0.3) (layer "F.Cu") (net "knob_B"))
 (segment (start 156.75 57.55) (end 156.8 57.55) (width 0.3) (layer "F.Cu") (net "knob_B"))
 (segment (start 155.464106 37.27) (end 152.54 37.27) (width 0.3) (layer "F.Cu") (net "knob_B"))
 (segment (start 156.75 59.9) (end 156.75 59.309189) (width 0.3) (layer "F.Cu") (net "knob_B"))
 (segment (start 152.36 37.946286) (end 152.4 37.986286) (width 0.3) (layer "F.Cu") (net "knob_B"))
 (segment (start 152.679576 39.86) (end 152.729576 39.81) (width 0.3) (layer "F.Cu") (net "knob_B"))
 (segment (start 153.279286 39.81) (end 154.467786 40.9985) (width 0.3) (layer "F.Cu") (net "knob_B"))
 (segment (start 156.75 38.626605) (end 156.192 38.068605) (width 0.3) (layer "F.Cu") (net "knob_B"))
 (segment (start 156.8 54.85) (end 156.75 54.85) (width 0.3) (layer "F.Cu") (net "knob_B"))
 (segment (start 152.54 37.27) (end 152.36 37.45) (width 0.3) (layer "F.Cu") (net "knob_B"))
 (segment (start 152.09 39.86) (end 152.679576 39.86) (width 0.3) (layer "F.Cu") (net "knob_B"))
 (segment (start 156.8 58.140811) (end 156.75 58.090811) (width 0.3) (layer "F.Cu") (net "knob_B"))
 (segment (start 172.02 40.1585) (end 170.32 38.4585) (width 0.3) (layer "B.Cu") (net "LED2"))
 (segment (start 172.02 47.23) (end 172.02 40.1585) (width 0.3) (layer "B.Cu") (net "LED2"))
 (segment (start 156.11 63.14) (end 172.02 47.23) (width 0.3) (layer "B.Cu") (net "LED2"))
 (segment (start 156.11 69.95) (end 156.11 63.14) (width 0.3) (layer "B.Cu") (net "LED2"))
 (segment (start 172.2485 35.9185) (end 170.32 35.9185) (width 0.3) (layer "B.Cu") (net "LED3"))
 (segment (start 175.05 38.72) (end 172.2485 35.9185) (width 0.3) (layer "B.Cu") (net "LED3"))
 (segment (start 175.05 69.97) (end 175.05 38.72) (width 0.3) (layer "B.Cu") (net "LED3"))
 (segment (start 156.11 75.03) (end 160.030508 75.03) (width 0.3) (layer "F.Cu") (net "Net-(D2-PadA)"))
 (segment (start 160.030508 75.03) (end 160.705508 74.355) (width 0.3) (layer "F.Cu") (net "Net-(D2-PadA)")))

